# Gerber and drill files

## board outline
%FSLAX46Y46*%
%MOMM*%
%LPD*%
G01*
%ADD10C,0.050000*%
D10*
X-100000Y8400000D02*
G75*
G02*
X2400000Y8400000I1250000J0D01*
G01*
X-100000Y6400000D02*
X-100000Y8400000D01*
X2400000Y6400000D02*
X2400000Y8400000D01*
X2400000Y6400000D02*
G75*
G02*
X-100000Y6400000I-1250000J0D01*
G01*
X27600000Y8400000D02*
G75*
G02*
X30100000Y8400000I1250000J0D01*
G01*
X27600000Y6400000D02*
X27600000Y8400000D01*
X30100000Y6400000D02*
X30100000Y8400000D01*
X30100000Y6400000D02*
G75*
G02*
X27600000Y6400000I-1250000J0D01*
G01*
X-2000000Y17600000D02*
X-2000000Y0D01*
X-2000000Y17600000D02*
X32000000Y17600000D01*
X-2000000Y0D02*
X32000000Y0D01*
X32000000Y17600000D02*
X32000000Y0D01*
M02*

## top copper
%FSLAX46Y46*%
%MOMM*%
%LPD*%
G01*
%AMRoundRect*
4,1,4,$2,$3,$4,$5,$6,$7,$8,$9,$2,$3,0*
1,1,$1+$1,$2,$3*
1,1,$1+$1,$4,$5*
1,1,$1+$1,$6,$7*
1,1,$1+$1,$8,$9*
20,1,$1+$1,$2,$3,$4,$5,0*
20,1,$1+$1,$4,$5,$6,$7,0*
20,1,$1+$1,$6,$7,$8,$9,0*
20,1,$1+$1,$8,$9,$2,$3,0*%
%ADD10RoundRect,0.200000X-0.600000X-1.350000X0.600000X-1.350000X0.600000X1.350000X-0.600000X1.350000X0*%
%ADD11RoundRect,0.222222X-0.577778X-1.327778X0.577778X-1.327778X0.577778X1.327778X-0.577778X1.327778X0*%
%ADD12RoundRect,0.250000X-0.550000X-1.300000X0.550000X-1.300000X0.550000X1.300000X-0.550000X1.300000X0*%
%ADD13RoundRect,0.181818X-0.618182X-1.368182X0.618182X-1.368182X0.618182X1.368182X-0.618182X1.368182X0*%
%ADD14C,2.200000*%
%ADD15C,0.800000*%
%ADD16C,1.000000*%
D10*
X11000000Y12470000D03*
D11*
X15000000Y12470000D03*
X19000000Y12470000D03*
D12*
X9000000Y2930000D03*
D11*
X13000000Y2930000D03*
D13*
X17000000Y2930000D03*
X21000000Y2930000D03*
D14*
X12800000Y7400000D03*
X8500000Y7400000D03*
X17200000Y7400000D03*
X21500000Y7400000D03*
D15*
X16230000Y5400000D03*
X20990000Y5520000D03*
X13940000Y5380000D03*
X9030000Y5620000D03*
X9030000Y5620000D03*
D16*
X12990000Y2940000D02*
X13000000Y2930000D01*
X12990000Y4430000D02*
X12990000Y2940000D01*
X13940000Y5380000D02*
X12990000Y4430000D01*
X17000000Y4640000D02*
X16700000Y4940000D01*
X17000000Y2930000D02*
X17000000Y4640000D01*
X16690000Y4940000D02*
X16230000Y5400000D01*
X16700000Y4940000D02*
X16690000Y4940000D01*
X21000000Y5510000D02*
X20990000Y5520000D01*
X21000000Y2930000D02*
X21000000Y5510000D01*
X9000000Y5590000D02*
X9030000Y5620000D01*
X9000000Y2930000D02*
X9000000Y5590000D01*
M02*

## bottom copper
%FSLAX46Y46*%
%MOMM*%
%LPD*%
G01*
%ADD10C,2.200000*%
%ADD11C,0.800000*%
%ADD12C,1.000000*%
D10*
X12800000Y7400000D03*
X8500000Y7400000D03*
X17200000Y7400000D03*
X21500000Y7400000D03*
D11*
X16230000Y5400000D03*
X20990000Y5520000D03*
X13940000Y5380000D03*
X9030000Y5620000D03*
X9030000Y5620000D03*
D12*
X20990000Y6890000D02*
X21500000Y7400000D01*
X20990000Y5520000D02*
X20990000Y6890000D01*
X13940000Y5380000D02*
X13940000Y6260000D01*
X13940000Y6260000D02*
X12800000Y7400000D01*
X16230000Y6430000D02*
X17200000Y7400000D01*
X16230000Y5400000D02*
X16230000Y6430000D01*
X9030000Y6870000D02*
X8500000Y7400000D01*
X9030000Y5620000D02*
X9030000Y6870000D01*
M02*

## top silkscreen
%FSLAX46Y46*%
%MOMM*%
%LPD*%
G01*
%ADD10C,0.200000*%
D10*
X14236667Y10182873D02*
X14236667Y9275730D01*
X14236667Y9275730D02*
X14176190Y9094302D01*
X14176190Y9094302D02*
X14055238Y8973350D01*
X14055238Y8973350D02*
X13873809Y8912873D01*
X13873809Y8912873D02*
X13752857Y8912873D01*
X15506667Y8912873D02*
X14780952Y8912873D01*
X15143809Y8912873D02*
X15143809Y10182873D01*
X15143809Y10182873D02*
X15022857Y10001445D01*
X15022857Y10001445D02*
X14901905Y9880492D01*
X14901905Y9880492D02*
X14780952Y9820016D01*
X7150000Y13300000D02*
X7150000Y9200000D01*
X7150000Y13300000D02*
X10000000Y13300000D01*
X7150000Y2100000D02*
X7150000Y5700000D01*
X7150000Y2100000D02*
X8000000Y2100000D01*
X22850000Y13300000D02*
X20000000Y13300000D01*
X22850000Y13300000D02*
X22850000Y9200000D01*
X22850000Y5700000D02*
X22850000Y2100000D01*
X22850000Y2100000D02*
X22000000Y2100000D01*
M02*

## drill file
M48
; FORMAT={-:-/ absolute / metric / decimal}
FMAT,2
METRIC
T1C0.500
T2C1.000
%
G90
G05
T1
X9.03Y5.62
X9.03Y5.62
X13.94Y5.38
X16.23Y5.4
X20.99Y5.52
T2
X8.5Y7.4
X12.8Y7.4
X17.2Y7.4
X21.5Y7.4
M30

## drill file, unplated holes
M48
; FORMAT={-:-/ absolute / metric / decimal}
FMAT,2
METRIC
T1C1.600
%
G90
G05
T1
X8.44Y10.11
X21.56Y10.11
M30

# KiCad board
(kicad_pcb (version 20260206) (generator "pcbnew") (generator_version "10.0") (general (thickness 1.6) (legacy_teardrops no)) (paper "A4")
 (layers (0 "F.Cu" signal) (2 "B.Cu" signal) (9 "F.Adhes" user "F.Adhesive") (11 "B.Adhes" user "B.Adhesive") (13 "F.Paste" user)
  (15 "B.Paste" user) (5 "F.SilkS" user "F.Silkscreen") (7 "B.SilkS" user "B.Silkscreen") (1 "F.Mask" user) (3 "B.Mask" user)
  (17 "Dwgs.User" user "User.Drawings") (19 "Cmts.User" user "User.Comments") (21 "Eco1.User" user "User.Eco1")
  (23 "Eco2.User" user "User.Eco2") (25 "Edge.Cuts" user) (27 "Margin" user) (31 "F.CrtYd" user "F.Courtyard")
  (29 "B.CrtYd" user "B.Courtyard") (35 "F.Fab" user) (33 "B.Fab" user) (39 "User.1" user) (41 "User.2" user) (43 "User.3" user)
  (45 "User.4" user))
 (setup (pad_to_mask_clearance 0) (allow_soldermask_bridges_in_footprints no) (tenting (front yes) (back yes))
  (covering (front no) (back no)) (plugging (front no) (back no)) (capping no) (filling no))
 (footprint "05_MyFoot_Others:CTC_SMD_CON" (layer "F.Cu") (at 15 -7.7)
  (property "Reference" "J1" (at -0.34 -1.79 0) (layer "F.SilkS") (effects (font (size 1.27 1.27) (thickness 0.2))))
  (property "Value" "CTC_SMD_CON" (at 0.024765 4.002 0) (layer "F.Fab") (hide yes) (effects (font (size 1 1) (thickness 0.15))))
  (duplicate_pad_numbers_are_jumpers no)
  (fp_line (start -7.85 -5.6) (end -7.85 -1.5) (stroke (width 0.2) (type solid)) (layer "F.SilkS"))
  (fp_line (start -7.85 -5.6) (end -5 -5.6) (stroke (width 0.2) (type solid)) (layer "F.SilkS"))
  (fp_line (start -7.85 5.6) (end -7.85 2) (stroke (width 0.2) (type solid)) (layer "F.SilkS"))
  (fp_line (start -7.85 5.6) (end -7 5.6) (stroke (width 0.2) (type solid)) (layer "F.SilkS"))
  (fp_line (start 7.85 -5.6) (end 5 -5.6) (stroke (width 0.2) (type solid)) (layer "F.SilkS"))
  (fp_line (start 7.85 -5.6) (end 7.85 -1.5) (stroke (width 0.2) (type solid)) (layer "F.SilkS"))
  (fp_line (start 7.85 2) (end 7.85 5.6) (stroke (width 0.2) (type solid)) (layer "F.SilkS"))
  (fp_line (start 7.85 5.6) (end 7 5.6) (stroke (width 0.2) (type solid)) (layer "F.SilkS"))
  (pad "" np_thru_hole circle (at -6.56 -2.41) (size 1.6 1.6) (drill 1.6) (layers "*.Cu") (thermal_bridge_angle 90))
  (pad "" np_thru_hole circle (at 6.56 -2.41) (size 1.6 1.6) (drill 1.6) (layers "*.Cu") (thermal_bridge_angle 90))
  (pad "1" smd roundrect (at -4 -4.77) (size 1.6 3.1) (layers "F.Cu" "F.Mask" "F.Paste") (roundrect_rratio 0.125)
   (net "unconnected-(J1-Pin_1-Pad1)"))
  (pad "2" smd roundrect (at 0 -4.77) (size 1.6 3.1) (layers "F.Cu" "F.Mask" "F.Paste") (roundrect_rratio 0.1388888889)
   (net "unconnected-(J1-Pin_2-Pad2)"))
  (pad "3" smd roundrect (at 4 -4.77) (size 1.6 3.1) (layers "F.Cu" "F.Mask" "F.Paste") (roundrect_rratio 0.1388888889)
   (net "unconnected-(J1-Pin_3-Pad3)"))
  (pad "4" smd roundrect (at -6 4.77) (size 1.6 3.1) (layers "F.Cu" "F.Mask" "F.Paste") (roundrect_rratio 0.15625) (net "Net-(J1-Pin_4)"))
  (pad "5" smd roundrect (at -2 4.77) (size 1.6 3.1) (layers "F.Cu" "F.Mask" "F.Paste") (roundrect_rratio 0.1388888889)
   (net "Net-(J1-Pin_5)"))
  (pad "6" smd roundrect (at 2 4.77) (size 1.6 3.1) (layers "F.Cu" "F.Mask" "F.Paste") (roundrect_rratio 0.1136363636)
   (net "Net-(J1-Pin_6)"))
  (pad "7" smd roundrect (at 6 4.77) (size 1.6 3.1) (layers "F.Cu" "F.Mask" "F.Paste") (roundrect_rratio 0.1136363636)
   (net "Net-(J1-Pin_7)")))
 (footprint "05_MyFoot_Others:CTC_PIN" (layer "B.Cu") (at 12.8 -7.4 180)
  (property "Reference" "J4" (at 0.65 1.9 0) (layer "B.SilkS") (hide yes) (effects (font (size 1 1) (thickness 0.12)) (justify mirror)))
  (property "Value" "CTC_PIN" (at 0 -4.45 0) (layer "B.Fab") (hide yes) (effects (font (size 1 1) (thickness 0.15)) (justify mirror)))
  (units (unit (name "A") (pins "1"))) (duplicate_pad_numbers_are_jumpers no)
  (pad "1" thru_hole circle (at 0 0 180) (size 2.2 2.2) (drill 1) (layers "*.Cu" "*.Mask") (remove_unused_layers no) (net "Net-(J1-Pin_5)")
   (zone_connect 2)))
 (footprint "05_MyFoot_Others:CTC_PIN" (layer "B.Cu") (at 8.5 -7.4 180)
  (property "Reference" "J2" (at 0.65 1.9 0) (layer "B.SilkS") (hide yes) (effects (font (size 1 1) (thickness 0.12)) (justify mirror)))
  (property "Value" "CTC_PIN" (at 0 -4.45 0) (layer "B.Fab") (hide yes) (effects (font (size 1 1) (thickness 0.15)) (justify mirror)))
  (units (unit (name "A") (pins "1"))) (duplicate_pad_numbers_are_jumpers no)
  (pad "1" thru_hole circle (at 0 0 180) (size 2.2 2.2) (drill 1) (layers "*.Cu" "*.Mask") (remove_unused_layers no) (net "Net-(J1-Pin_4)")
   (zone_connect 2)))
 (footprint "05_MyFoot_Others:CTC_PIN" (layer "B.Cu") (at 17.2 -7.4 180)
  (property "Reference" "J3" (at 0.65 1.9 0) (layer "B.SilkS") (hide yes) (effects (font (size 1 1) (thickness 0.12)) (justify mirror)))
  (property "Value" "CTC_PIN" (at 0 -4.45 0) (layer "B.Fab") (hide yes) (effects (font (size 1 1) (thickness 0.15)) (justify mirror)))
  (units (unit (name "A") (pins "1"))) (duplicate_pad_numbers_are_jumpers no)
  (pad "1" thru_hole circle (at 0 0 180) (size 2.2 2.2) (drill 1) (layers "*.Cu" "*.Mask") (remove_unused_layers no) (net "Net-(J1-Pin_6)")
   (zone_connect 2)))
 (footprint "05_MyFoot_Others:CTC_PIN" (layer "B.Cu") (at 21.5 -7.4 180)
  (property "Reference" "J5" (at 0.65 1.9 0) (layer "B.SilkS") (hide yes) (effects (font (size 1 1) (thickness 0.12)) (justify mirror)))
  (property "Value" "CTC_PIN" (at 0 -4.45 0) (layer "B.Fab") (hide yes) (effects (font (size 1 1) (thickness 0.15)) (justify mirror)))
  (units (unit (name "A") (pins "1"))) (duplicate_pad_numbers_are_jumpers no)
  (pad "1" thru_hole circle (at 0 0 180) (size 2.2 2.2) (drill 1) (layers "*.Cu" "*.Mask") (remove_unused_layers no) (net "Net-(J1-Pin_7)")
   (zone_connect 2)))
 (gr_line (start -2 -17.6) (end -2 0) (stroke (width 0.05) (type default)) (layer "Edge.Cuts"))
 (gr_line (start -2 -17.6) (end 32 -17.6) (stroke (width 0.05) (type solid)) (layer "Edge.Cuts"))
 (gr_line (start -2 0) (end 32 0) (stroke (width 0.05) (type solid)) (layer "Edge.Cuts"))
 (gr_arc (start -0.1 -8.4) (mid 1.15 -9.65) (end 2.4 -8.4) (stroke (width 0.05) (type solid)) (layer "Edge.Cuts"))
 (gr_line (start -0.1 -6.4) (end -0.1 -8.4) (stroke (width 0.05) (type solid)) (layer "Edge.Cuts"))
 (gr_arc (start 2.4 -6.4) (mid 1.15 -5.15) (end -0.1 -6.4) (stroke (width 0.05) (type solid)) (layer "Edge.Cuts"))
 (gr_line (start 2.4 -6.4) (end 2.4 -8.4) (stroke (width 0.05) (type solid)) (layer "Edge.Cuts"))
 (gr_arc (start 27.6 -8.4) (mid 28.85 -9.65) (end 30.1 -8.4) (stroke (width 0.05) (type solid)) (layer "Edge.Cuts"))
 (gr_line (start 27.6 -6.4) (end 27.6 -8.4) (stroke (width 0.05) (type solid)) (layer "Edge.Cuts"))
 (gr_arc (start 30.1 -6.4) (mid 28.85 -5.15) (end 27.6 -6.4) (stroke (width 0.05) (type solid)) (layer "Edge.Cuts"))
 (gr_line (start 30.1 -6.4) (end 30.1 -8.4) (stroke (width 0.05) (type solid)) (layer "Edge.Cuts"))
 (gr_line (start 32 -17.6) (end 32 0) (stroke (width 0.05) (type default)) (layer "Edge.Cuts"))
 (segment (start 9 -5.59) (end 9.03 -5.62) (width 1) (layer "F.Cu") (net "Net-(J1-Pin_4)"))
 (segment (start 9 -2.93) (end 9 -5.59) (width 1) (layer "F.Cu") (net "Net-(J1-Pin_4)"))
 (via (at 9.03 -5.62) (size 0.8) (drill 0.5) (layers "F.Cu" "B.Cu") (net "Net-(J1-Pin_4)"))
 (via (at 9.03 -5.62) (size 0.8) (drill 0.5) (layers "F.Cu" "B.Cu") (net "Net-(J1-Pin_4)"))
 (segment (start 9.03 -5.62) (end 9.03 -6.87) (width 1) (layer "B.Cu") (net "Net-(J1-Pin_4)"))
 (segment (start 9.03 -6.87) (end 8.5 -7.4) (width 1) (layer "B.Cu") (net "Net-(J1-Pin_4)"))
 (segment (start 12.99 -2.94) (end 13 -2.93) (width 1) (layer "F.Cu") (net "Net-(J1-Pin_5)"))
 (segment (start 13.94 -5.38) (end 12.99 -4.43) (width 1) (layer "F.Cu") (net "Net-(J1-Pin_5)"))
 (segment (start 12.99 -4.43) (end 12.99 -2.94) (width 1) (layer "F.Cu") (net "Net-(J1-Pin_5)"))
 (via (at 13.94 -5.38) (size 0.8) (drill 0.5) (layers "F.Cu" "B.Cu") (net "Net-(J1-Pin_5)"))
 (segment (start 13.94 -5.38) (end 13.94 -6.26) (width 1) (layer "B.Cu") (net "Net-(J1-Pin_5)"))
 (segment (start 13.94 -6.26) (end 12.8 -7.4) (width 1) (layer "B.Cu") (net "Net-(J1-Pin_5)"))
 (segment (start 17 -4.64) (end 16.7 -4.94) (width 1) (layer "F.Cu") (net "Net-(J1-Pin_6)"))
 (segment (start 17 -2.93) (end 17 -4.64) (width 1) (layer "F.Cu") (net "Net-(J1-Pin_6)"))
 (segment (start 16.69 -4.94) (end 16.23 -5.4) (width 1) (layer "F.Cu") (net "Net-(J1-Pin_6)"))
 (segment (start 16.7 -4.94) (end 16.69 -4.94) (width 1) (layer "F.Cu") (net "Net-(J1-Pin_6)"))
 (via (at 16.23 -5.4) (size 0.8) (drill 0.5) (layers "F.Cu" "B.Cu") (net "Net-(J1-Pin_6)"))
 (segment (start 16.23 -6.43) (end 17.2 -7.4) (width 1) (layer "B.Cu") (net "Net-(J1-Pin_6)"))
 (segment (start 16.23 -5.4) (end 16.23 -6.43) (width 1) (layer "B.Cu") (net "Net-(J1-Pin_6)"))
 (segment (start 21 -5.51) (end 20.99 -5.52) (width 1) (layer "F.Cu") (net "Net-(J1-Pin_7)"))
 (segment (start 21 -2.93) (end 21 -5.51) (width 1) (layer "F.Cu") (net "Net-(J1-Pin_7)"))
 (via (at 20.99 -5.52) (size 0.8) (drill 0.5) (layers "F.Cu" "B.Cu") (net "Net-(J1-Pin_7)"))
 (segment (start 20.99 -5.52) (end 20.99 -6.89) (width 1) (layer "B.Cu") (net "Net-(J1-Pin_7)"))
 (segment (start 20.99 -6.89) (end 21.5 -7.4) (width 1) (layer "B.Cu") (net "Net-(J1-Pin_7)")))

